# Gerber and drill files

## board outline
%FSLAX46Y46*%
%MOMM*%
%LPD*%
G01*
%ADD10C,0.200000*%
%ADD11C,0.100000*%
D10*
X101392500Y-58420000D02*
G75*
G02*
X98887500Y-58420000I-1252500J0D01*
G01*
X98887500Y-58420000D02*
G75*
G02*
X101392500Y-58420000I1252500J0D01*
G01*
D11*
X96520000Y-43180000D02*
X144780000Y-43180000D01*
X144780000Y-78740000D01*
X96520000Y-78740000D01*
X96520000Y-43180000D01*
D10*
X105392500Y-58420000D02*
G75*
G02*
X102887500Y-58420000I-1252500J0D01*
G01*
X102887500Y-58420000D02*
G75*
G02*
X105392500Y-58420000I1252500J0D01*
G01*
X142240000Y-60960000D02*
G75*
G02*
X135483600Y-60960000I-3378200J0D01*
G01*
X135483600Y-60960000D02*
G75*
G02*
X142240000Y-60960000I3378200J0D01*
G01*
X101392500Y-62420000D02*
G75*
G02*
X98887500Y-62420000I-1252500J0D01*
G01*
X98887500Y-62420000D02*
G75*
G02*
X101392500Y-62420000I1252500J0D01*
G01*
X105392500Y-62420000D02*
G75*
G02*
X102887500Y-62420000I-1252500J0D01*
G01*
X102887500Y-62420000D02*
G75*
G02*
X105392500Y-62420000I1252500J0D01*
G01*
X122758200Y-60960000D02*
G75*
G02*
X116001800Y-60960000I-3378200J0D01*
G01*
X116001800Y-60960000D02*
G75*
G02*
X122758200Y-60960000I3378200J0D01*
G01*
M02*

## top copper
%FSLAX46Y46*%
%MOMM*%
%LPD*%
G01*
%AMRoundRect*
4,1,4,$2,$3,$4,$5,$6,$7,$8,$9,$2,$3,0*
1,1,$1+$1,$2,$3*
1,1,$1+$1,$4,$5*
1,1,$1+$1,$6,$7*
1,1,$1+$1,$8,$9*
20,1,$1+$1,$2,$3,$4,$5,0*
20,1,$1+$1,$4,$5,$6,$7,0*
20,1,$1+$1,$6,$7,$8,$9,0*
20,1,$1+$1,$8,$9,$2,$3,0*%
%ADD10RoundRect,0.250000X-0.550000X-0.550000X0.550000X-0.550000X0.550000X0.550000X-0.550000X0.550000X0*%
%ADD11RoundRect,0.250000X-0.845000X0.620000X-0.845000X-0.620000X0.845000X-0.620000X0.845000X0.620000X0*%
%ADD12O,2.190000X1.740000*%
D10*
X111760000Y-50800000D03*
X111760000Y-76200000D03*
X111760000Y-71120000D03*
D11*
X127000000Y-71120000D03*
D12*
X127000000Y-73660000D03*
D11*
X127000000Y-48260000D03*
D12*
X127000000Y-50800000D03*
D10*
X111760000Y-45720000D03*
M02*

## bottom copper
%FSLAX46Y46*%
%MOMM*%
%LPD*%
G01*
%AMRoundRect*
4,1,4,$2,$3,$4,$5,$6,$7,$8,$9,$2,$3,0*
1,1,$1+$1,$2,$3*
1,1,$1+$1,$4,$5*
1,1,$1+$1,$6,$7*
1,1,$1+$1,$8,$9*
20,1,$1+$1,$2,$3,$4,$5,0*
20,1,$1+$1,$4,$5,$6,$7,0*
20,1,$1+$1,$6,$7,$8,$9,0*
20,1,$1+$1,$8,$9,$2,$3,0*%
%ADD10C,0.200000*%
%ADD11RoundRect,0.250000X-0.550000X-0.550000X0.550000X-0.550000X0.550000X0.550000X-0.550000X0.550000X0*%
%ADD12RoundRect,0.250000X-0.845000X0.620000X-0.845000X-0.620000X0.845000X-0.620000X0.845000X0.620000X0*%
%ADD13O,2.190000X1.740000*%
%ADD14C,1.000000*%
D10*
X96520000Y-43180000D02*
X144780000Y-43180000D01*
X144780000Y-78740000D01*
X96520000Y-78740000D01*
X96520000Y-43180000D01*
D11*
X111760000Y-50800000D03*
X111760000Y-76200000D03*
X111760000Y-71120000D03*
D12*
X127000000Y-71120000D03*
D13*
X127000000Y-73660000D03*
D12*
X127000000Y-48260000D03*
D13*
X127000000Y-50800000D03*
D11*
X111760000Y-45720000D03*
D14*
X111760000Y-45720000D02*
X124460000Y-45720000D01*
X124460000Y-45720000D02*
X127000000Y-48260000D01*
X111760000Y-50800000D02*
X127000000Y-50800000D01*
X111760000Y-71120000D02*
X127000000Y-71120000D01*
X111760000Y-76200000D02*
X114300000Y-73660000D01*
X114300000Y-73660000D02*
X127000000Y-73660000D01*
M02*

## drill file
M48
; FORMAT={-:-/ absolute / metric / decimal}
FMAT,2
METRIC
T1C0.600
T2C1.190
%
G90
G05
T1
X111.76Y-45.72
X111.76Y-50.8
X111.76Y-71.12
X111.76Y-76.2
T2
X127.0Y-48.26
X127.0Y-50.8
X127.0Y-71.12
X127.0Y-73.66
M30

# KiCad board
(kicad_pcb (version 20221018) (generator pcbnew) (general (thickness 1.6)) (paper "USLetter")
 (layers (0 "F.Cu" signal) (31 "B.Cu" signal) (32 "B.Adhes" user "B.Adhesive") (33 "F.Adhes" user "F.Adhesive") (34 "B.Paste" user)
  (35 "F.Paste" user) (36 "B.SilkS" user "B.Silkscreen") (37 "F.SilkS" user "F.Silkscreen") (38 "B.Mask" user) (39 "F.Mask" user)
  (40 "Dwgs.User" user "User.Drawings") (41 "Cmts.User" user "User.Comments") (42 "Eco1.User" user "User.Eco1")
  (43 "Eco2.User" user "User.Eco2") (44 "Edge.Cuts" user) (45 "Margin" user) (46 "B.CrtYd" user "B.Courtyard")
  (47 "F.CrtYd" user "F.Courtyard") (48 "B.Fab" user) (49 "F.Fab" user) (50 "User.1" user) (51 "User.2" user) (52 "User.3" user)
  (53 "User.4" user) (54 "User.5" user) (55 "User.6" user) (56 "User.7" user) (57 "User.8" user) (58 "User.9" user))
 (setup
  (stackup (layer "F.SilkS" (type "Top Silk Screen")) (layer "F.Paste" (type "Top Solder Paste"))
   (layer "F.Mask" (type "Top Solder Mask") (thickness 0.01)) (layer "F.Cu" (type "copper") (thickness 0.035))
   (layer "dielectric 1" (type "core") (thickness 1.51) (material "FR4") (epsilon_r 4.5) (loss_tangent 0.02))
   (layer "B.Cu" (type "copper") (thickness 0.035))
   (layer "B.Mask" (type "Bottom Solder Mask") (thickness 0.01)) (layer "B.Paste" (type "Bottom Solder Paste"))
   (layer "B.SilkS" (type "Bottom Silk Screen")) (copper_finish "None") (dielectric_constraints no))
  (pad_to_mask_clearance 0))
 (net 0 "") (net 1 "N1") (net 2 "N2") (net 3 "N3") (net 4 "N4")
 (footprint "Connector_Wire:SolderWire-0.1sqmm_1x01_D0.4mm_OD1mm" (layer "F.Cu") (at 111.76 50.8)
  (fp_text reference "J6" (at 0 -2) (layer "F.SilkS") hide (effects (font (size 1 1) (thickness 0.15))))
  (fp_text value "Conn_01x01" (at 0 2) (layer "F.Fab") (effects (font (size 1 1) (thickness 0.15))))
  (pad "1" thru_hole roundrect (at 0 0) (size 1.6 1.6) (drill 0.6) (layers "*.Cu" "*.Mask") (roundrect_rratio 0.15625) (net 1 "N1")))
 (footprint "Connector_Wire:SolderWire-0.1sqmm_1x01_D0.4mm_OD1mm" (layer "F.Cu") (at 111.76 76.2)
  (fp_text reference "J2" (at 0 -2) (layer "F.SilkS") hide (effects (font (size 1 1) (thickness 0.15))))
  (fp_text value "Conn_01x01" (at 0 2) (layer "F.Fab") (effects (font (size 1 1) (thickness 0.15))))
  (pad "1" thru_hole roundrect (at 0 0) (size 1.6 1.6) (drill 0.6) (layers "*.Cu" "*.Mask") (roundrect_rratio 0.15625) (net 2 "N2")))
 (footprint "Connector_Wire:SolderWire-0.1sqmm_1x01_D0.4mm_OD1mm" (layer "F.Cu") (at 111.76 71.12)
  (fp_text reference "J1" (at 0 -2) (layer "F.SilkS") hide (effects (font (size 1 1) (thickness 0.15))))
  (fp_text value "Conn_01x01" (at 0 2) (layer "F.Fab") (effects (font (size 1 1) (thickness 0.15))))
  (pad "1" thru_hole roundrect (at 0 0) (size 1.6 1.6) (drill 0.6) (layers "*.Cu" "*.Mask") (roundrect_rratio 0.15625) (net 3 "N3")))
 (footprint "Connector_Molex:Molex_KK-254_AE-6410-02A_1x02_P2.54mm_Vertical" (layer "F.Cu") (at 127 71.12 -90)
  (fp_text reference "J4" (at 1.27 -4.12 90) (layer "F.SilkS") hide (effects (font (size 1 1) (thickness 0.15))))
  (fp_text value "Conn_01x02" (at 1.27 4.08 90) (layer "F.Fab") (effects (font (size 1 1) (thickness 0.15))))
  (pad "1" thru_hole roundrect (at 0 0 270) (size 1.74 2.19) (drill 1.19) (layers "*.Cu" "*.Mask") (roundrect_rratio 0.1436781609)
   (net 3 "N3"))
  (pad "2" thru_hole oval (at 2.54 0 270) (size 1.74 2.19) (drill 1.19) (layers "*.Cu" "*.Mask") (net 2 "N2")))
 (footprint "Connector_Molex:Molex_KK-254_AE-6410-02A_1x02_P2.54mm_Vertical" (layer "F.Cu") (at 127 48.26 -90)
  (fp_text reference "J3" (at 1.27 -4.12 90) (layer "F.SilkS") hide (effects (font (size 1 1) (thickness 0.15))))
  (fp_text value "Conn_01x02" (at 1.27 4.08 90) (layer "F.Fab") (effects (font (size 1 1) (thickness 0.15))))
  (pad "1" thru_hole roundrect (at 0 0 270) (size 1.74 2.19) (drill 1.19) (layers "*.Cu" "*.Mask") (roundrect_rratio 0.1436781609)
   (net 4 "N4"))
  (pad "2" thru_hole oval (at 2.54 0 270) (size 1.74 2.19) (drill 1.19) (layers "*.Cu" "*.Mask") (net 1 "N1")))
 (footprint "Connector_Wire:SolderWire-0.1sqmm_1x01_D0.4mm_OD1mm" (layer "F.Cu") (at 111.76 45.72)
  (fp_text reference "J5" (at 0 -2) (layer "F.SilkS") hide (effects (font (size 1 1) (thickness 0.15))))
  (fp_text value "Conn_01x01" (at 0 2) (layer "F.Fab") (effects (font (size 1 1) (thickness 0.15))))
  (pad "1" thru_hole roundrect (at 0 0) (size 1.6 1.6) (drill 0.6) (layers "*.Cu" "*.Mask") (roundrect_rratio 0.15625) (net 4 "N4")))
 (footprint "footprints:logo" (layer "F.Cu") (at 129.032 60.96 90)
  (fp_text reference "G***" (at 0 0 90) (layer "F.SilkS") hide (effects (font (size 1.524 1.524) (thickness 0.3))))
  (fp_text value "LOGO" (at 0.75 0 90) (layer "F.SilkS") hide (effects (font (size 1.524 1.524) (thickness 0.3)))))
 (gr_rect (start 96.52 43.18) (end 144.78 78.74) (stroke (width 0.2) (type solid)) (fill none) (layer "B.Cu"))
 (gr_circle (center 100.14 58.42) (end 101.3925 58.42) (stroke (width 0.2) (type solid)) (fill none) (layer "Edge.Cuts"))
 (gr_rect (start 96.52 43.18) (end 144.78 78.74) (stroke (width 0.1) (type default)) (fill none) (layer "Edge.Cuts"))
 (gr_circle (center 104.14 58.42) (end 105.3925 58.42) (stroke (width 0.2) (type solid)) (fill none) (layer "Edge.Cuts"))
 (gr_circle (center 138.8618 60.96) (end 142.24 60.96) (stroke (width 0.2) (type solid)) (fill none) (layer "Edge.Cuts"))
 (gr_circle (center 100.14 62.42) (end 101.3925 62.42) (stroke (width 0.2) (type solid)) (fill none) (layer "Edge.Cuts"))
 (gr_circle (center 104.14 62.42) (end 105.3925 62.42) (stroke (width 0.2) (type solid)) (fill none) (layer "Edge.Cuts"))
 (gr_circle (center 119.38 60.96) (end 122.7582 60.96) (stroke (width 0.2) (type solid)) (fill none) (layer "Edge.Cuts"))
 (segment (start 111.76 45.72) (end 124.46 45.72) (width 1) (layer "B.Cu") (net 4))
 (segment (start 124.46 45.72) (end 127 48.26) (width 1) (layer "B.Cu") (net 4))
 (segment (start 111.76 50.8) (end 127 50.8) (width 1) (layer "B.Cu") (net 1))
 (segment (start 111.76 71.12) (end 127 71.12) (width 1) (layer "B.Cu") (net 3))
 (segment (start 111.76 76.2) (end 114.3 73.66) (width 1) (layer "B.Cu") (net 2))
 (segment (start 114.3 73.66) (end 127 73.66) (width 1) (layer "B.Cu") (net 2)))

